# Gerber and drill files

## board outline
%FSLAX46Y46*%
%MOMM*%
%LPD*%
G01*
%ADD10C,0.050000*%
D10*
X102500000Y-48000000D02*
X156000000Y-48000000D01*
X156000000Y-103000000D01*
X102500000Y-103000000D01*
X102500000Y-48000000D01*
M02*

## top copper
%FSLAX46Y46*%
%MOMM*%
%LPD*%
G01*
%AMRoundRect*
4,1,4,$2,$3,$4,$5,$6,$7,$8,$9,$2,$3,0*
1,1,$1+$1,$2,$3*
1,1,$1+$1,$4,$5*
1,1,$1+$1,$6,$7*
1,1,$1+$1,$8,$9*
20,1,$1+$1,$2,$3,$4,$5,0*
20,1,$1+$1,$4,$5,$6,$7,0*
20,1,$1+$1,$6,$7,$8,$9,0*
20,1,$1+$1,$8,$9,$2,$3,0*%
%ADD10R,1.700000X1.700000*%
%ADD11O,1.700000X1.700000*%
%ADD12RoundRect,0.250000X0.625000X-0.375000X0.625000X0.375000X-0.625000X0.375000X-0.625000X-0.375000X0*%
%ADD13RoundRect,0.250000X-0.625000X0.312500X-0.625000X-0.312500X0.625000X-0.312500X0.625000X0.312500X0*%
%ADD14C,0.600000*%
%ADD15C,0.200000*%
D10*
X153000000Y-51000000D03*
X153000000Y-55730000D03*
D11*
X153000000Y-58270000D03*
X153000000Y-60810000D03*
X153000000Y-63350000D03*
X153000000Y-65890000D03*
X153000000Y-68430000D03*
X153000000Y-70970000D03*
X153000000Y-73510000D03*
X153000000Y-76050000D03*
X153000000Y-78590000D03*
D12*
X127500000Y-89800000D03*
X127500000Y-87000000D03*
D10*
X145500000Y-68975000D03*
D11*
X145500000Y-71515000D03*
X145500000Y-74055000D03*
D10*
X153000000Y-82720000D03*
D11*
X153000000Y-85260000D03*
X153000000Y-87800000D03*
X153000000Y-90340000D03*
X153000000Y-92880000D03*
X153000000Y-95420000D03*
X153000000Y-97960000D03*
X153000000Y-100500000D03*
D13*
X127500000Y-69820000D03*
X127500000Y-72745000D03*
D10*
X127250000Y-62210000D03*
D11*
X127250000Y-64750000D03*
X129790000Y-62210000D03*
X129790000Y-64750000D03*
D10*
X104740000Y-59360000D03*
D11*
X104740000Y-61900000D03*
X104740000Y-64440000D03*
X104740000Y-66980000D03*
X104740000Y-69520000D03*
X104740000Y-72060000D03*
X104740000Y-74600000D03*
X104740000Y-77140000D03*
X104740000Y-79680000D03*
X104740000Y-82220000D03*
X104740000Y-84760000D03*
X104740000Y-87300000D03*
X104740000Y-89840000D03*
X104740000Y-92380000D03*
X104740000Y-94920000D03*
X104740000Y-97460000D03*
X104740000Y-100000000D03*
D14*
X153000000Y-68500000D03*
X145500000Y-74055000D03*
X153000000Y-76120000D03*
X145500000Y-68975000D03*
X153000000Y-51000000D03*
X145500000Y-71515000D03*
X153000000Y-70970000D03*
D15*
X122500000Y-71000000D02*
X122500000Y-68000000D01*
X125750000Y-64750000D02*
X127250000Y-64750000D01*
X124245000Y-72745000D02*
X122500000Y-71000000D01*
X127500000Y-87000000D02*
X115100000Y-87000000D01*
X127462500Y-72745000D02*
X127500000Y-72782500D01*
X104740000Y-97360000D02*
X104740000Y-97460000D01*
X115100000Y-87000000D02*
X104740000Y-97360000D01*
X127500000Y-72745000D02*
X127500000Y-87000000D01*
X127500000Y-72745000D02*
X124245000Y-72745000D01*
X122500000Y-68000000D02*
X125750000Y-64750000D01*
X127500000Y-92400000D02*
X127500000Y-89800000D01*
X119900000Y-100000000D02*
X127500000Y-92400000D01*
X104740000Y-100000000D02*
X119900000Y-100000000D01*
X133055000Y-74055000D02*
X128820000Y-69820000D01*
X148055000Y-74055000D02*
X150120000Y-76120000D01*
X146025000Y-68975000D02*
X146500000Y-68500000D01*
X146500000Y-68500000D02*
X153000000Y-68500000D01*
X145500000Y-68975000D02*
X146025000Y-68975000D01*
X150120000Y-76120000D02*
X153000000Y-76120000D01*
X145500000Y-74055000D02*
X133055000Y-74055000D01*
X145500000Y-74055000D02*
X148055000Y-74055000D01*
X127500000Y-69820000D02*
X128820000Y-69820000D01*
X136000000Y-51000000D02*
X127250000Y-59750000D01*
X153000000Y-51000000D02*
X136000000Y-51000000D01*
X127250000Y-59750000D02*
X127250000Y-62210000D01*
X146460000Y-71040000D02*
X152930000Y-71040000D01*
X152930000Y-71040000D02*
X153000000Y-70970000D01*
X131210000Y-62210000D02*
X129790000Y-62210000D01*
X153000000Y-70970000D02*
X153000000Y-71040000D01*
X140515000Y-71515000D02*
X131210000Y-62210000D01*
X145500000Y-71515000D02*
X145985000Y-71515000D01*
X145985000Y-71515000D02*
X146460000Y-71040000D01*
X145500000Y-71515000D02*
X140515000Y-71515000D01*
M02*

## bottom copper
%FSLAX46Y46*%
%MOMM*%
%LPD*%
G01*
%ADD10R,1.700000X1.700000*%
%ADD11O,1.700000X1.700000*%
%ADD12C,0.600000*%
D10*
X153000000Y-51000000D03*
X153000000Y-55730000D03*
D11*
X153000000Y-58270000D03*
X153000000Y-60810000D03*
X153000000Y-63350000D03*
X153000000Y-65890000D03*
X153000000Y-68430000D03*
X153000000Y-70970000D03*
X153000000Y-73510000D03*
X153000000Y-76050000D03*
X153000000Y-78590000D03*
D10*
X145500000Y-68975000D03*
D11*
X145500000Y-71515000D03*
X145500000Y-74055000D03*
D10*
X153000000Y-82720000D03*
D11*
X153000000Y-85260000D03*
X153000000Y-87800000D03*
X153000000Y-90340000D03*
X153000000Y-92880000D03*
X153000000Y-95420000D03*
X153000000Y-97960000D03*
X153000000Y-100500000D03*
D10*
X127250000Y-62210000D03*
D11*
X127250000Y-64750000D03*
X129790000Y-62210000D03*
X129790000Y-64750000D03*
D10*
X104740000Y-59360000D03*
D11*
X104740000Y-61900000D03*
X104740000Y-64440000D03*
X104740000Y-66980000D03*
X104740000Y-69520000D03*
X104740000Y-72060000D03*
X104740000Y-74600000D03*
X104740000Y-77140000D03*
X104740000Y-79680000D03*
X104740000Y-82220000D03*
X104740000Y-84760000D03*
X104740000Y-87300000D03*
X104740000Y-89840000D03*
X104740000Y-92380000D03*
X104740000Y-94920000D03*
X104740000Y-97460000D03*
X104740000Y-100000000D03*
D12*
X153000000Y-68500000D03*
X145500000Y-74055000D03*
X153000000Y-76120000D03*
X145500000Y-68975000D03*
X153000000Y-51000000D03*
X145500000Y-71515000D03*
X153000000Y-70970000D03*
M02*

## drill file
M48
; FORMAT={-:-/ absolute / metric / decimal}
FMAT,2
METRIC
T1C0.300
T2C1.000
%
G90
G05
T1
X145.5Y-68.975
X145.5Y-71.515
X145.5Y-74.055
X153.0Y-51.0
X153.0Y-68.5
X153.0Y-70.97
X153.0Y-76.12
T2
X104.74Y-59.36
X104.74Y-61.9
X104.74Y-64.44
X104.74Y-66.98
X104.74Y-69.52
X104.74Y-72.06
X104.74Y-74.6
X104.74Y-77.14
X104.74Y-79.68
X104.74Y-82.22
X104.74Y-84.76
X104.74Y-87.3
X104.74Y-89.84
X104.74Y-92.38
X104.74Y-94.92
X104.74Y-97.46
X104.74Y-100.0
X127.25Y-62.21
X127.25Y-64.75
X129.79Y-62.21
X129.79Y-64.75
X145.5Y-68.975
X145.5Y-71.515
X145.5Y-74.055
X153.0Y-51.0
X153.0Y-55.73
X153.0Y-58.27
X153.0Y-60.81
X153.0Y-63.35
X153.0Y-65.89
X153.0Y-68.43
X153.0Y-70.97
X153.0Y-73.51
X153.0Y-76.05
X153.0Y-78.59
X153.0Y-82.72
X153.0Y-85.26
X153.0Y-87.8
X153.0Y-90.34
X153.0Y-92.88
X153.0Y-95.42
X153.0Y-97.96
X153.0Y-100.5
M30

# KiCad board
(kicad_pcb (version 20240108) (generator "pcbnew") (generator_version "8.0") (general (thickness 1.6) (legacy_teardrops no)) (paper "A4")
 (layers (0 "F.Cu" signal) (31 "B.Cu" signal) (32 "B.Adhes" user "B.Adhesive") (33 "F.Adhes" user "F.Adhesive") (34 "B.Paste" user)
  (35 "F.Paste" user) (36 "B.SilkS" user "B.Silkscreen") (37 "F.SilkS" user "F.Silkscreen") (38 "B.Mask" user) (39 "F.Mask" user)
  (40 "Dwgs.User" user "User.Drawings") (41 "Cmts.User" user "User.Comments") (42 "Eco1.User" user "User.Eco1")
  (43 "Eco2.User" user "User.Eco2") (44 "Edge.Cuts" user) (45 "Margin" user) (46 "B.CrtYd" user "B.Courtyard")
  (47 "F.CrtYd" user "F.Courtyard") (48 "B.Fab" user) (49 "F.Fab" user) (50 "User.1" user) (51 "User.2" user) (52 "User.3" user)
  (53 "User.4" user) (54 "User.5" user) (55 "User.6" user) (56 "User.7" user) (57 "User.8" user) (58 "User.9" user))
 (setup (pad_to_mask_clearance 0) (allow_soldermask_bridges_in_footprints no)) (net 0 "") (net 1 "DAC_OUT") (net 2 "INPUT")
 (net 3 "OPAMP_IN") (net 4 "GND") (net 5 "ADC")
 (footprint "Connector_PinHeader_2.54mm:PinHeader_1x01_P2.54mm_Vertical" (layer "F.Cu") (at 153 51)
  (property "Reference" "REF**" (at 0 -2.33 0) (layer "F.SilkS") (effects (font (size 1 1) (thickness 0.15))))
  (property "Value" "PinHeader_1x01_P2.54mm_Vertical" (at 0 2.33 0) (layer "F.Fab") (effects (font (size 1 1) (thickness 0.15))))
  (pad "1" thru_hole rect (at 0 0) (size 1.7 1.7) (drill 1) (layers "*.Cu" "*.Mask") (remove_unused_layers no) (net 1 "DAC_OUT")))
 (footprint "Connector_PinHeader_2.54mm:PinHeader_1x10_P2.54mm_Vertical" (layer "F.Cu") (at 153 55.73)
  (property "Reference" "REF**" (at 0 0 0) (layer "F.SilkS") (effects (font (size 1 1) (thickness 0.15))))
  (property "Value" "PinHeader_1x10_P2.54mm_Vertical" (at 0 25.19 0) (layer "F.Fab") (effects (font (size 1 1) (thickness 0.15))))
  (pad "1" thru_hole rect (at 0 0) (size 1.7 1.7) (drill 1) (layers "*.Cu" "*.Mask") (remove_unused_layers no))
  (pad "2" thru_hole oval (at 0 2.54) (size 1.7 1.7) (drill 1) (layers "*.Cu" "*.Mask") (remove_unused_layers no))
  (pad "3" thru_hole oval (at 0 5.08) (size 1.7 1.7) (drill 1) (layers "*.Cu" "*.Mask") (remove_unused_layers no))
  (pad "4" thru_hole oval (at 0 7.62) (size 1.7 1.7) (drill 1) (layers "*.Cu" "*.Mask") (remove_unused_layers no))
  (pad "5" thru_hole oval (at 0 10.16) (size 1.7 1.7) (drill 1) (layers "*.Cu" "*.Mask") (remove_unused_layers no))
  (pad "6" thru_hole oval (at 0 12.7) (size 1.7 1.7) (drill 1) (layers "*.Cu" "*.Mask") (remove_unused_layers no) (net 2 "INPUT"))
  (pad "7" thru_hole oval (at 0 15.24) (size 1.7 1.7) (drill 1) (layers "*.Cu" "*.Mask") (remove_unused_layers no) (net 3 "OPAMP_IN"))
  (pad "8" thru_hole oval (at 0 17.78) (size 1.7 1.7) (drill 1) (layers "*.Cu" "*.Mask") (remove_unused_layers no))
  (pad "9" thru_hole oval (at 0 20.32) (size 1.7 1.7) (drill 1) (layers "*.Cu" "*.Mask") (remove_unused_layers no) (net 2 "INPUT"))
  (pad "10" thru_hole oval (at 0 22.86) (size 1.7 1.7) (drill 1) (layers "*.Cu" "*.Mask") (remove_unused_layers no)))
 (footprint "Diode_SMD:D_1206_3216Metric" (layer "F.Cu") (at 127.5 88.4 90)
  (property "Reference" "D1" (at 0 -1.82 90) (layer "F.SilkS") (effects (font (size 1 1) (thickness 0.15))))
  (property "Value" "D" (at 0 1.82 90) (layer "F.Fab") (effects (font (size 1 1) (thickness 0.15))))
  (pad "1" smd roundrect (at -1.4 0 90) (size 1.25 1.75) (layers "F.Cu" "F.Paste" "F.Mask") (roundrect_rratio 0.2) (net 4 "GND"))
  (pad "2" smd roundrect (at 1.4 0 90) (size 1.25 1.75) (layers "F.Cu" "F.Paste" "F.Mask") (roundrect_rratio 0.2) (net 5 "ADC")))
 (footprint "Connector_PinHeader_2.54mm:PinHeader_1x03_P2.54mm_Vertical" (layer "F.Cu") (at 145.5 68.975)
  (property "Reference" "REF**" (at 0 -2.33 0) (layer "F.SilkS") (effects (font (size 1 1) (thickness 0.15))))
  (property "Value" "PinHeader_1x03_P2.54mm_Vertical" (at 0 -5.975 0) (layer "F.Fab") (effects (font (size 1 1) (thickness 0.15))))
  (pad "1" thru_hole rect (at 0 0) (size 1.7 1.7) (drill 1) (layers "*.Cu" "*.Mask") (remove_unused_layers no) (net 2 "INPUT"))
  (pad "2" thru_hole oval (at 0 2.54) (size 1.7 1.7) (drill 1) (layers "*.Cu" "*.Mask") (remove_unused_layers no) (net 3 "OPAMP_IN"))
  (pad "3" thru_hole oval (at 0 5.08) (size 1.7 1.7) (drill 1) (layers "*.Cu" "*.Mask") (remove_unused_layers no) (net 2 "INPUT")))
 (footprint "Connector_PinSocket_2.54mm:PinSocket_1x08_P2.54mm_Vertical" (layer "F.Cu") (at 153 82.72)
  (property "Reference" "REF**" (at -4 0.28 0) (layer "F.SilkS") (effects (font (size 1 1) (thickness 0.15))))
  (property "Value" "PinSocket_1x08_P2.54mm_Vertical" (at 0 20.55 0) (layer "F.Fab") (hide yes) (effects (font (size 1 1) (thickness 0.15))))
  (pad "1" thru_hole rect (at 0 0) (size 1.7 1.7) (drill 1) (layers "*.Cu" "*.Mask") (remove_unused_layers no))
  (pad "2" thru_hole oval (at 0 2.54) (size 1.7 1.7) (drill 1) (layers "*.Cu" "*.Mask") (remove_unused_layers no))
  (pad "3" thru_hole oval (at 0 5.08) (size 1.7 1.7) (drill 1) (layers "*.Cu" "*.Mask") (remove_unused_layers no))
  (pad "4" thru_hole oval (at 0 7.62) (size 1.7 1.7) (drill 1) (layers "*.Cu" "*.Mask") (remove_unused_layers no))
  (pad "5" thru_hole oval (at 0 10.16) (size 1.7 1.7) (drill 1) (layers "*.Cu" "*.Mask") (remove_unused_layers no))
  (pad "6" thru_hole oval (at 0 12.7) (size 1.7 1.7) (drill 1) (layers "*.Cu" "*.Mask") (remove_unused_layers no))
  (pad "7" thru_hole oval (at 0 15.24) (size 1.7 1.7) (drill 1) (layers "*.Cu" "*.Mask") (remove_unused_layers no))
  (pad "8" thru_hole oval (at 0 17.78) (size 1.7 1.7) (drill 1) (layers "*.Cu" "*.Mask") (remove_unused_layers no)))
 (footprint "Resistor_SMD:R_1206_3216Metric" (layer "F.Cu") (at 127.5 71.2825 -90)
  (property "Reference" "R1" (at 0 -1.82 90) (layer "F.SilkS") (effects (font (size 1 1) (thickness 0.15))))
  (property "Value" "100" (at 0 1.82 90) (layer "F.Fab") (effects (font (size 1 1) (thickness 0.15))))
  (pad "1" smd roundrect (at -1.4625 0 270) (size 1.125 1.75) (layers "F.Cu" "F.Paste" "F.Mask") (roundrect_rratio 0.222222) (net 2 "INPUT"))
  (pad "2" smd roundrect (at 1.4625 0 270) (size 1.125 1.75) (layers "F.Cu" "F.Paste" "F.Mask") (roundrect_rratio 0.222222) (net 5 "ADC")))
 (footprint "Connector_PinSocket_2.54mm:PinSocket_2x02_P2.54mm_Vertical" (layer "F.Cu") (at 127.25 62.21 90)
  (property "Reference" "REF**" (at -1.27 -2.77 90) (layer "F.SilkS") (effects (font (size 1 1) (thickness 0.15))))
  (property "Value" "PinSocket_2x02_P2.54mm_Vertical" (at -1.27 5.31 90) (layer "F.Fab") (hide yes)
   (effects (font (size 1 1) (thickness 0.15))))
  (pad "1" thru_hole rect (at 0 0 90) (size 1.7 1.7) (drill 1) (layers "*.Cu" "*.Mask") (remove_unused_layers no) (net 1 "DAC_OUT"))
  (pad "2" thru_hole oval (at -2.54 0 90) (size 1.7 1.7) (drill 1) (layers "*.Cu" "*.Mask") (remove_unused_layers no) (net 5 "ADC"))
  (pad "3" thru_hole oval (at 0 2.54 90) (size 1.7 1.7) (drill 1) (layers "*.Cu" "*.Mask") (remove_unused_layers no) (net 3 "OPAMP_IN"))
  (pad "4" thru_hole oval (at -2.54 2.54 90) (size 1.7 1.7) (drill 1) (layers "*.Cu" "*.Mask") (remove_unused_layers no)))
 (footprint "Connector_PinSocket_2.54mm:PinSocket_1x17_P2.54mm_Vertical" (layer "F.Cu") (at 104.74 59.36)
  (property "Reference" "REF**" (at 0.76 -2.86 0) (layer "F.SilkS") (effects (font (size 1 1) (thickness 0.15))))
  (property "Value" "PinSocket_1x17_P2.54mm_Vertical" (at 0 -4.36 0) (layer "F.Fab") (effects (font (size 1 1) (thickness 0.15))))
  (pad "1" thru_hole rect (at 0 0) (size 1.7 1.7) (drill 1) (layers "*.Cu" "*.Mask") (remove_unused_layers no))
  (pad "2" thru_hole oval (at 0 2.54) (size 1.7 1.7) (drill 1) (layers "*.Cu" "*.Mask") (remove_unused_layers no))
  (pad "3" thru_hole oval (at 0 5.08) (size 1.7 1.7) (drill 1) (layers "*.Cu" "*.Mask") (remove_unused_layers no))
  (pad "4" thru_hole oval (at 0 7.62) (size 1.7 1.7) (drill 1) (layers "*.Cu" "*.Mask") (remove_unused_layers no))
  (pad "5" thru_hole oval (at 0 10.16) (size 1.7 1.7) (drill 1) (layers "*.Cu" "*.Mask") (remove_unused_layers no))
  (pad "6" thru_hole oval (at 0 12.7) (size 1.7 1.7) (drill 1) (layers "*.Cu" "*.Mask") (remove_unused_layers no))
  (pad "7" thru_hole oval (at 0 15.24) (size 1.7 1.7) (drill 1) (layers "*.Cu" "*.Mask") (remove_unused_layers no))
  (pad "8" thru_hole oval (at 0 17.78) (size 1.7 1.7) (drill 1) (layers "*.Cu" "*.Mask") (remove_unused_layers no))
  (pad "9" thru_hole oval (at 0 20.32) (size 1.7 1.7) (drill 1) (layers "*.Cu" "*.Mask") (remove_unused_layers no))
  (pad "10" thru_hole oval (at 0 22.86) (size 1.7 1.7) (drill 1) (layers "*.Cu" "*.Mask") (remove_unused_layers no))
  (pad "11" thru_hole oval (at 0 25.4) (size 1.7 1.7) (drill 1) (layers "*.Cu" "*.Mask") (remove_unused_layers no))
  (pad "12" thru_hole oval (at 0 27.94) (size 1.7 1.7) (drill 1) (layers "*.Cu" "*.Mask") (remove_unused_layers no))
  (pad "13" thru_hole oval (at 0 30.48) (size 1.7 1.7) (drill 1) (layers "*.Cu" "*.Mask") (remove_unused_layers no))
  (pad "14" thru_hole oval (at 0 33.02) (size 1.7 1.7) (drill 1) (layers "*.Cu" "*.Mask") (remove_unused_layers no))
  (pad "15" thru_hole oval (at 0 35.56) (size 1.7 1.7) (drill 1) (layers "*.Cu" "*.Mask") (remove_unused_layers no))
  (pad "16" thru_hole oval (at 0 38.1) (size 1.7 1.7) (drill 1) (layers "*.Cu" "*.Mask") (remove_unused_layers no) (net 5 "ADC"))
  (pad "17" thru_hole oval (at 0 40.64) (size 1.7 1.7) (drill 1) (layers "*.Cu" "*.Mask") (remove_unused_layers no) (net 4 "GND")))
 (gr_rect (start 102.5 48) (end 156 103) (stroke (width 0.05) (type default)) (fill none) (layer "Edge.Cuts"))
 (segment (start 122.5 71) (end 122.5 68) (width 0.2) (layer "F.Cu") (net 5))
 (segment (start 125.75 64.75) (end 127.25 64.75) (width 0.2) (layer "F.Cu") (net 5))
 (segment (start 124.245 72.745) (end 122.5 71) (width 0.2) (layer "F.Cu") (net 5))
 (segment (start 127.5 87) (end 115.1 87) (width 0.2) (layer "F.Cu") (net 5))
 (segment (start 127.4625 72.745) (end 127.5 72.7825) (width 0.2) (layer "F.Cu") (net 5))
 (segment (start 104.74 97.36) (end 104.74 97.46) (width 0.2) (layer "F.Cu") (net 5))
 (segment (start 115.1 87) (end 104.74 97.36) (width 0.2) (layer "F.Cu") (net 5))
 (segment (start 127.5 72.745) (end 127.5 87) (width 0.2) (layer "F.Cu") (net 5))
 (segment (start 127.5 72.745) (end 124.245 72.745) (width 0.2) (layer "F.Cu") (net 5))
 (segment (start 122.5 68) (end 125.75 64.75) (width 0.2) (layer "F.Cu") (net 5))
 (segment (start 127.5 92.4) (end 127.5 89.8) (width 0.2) (layer "F.Cu") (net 4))
 (segment (start 119.9 100) (end 127.5 92.4) (width 0.2) (layer "F.Cu") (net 4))
 (segment (start 104.74 100) (end 119.9 100) (width 0.2) (layer "F.Cu") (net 4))
 (segment (start 133.055 74.055) (end 128.82 69.82) (width 0.2) (layer "F.Cu") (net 2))
 (segment (start 148.055 74.055) (end 150.12 76.12) (width 0.2) (layer "F.Cu") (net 2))
 (segment (start 146.025 68.975) (end 146.5 68.5) (width 0.2) (layer "F.Cu") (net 2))
 (segment (start 146.5 68.5) (end 153 68.5) (width 0.2) (layer "F.Cu") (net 2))
 (segment (start 145.5 68.975) (end 146.025 68.975) (width 0.2) (layer "F.Cu") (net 2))
 (segment (start 150.12 76.12) (end 153 76.12) (width 0.2) (layer "F.Cu") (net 2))
 (segment (start 145.5 74.055) (end 133.055 74.055) (width 0.2) (layer "F.Cu") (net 2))
 (segment (start 145.5 74.055) (end 148.055 74.055) (width 0.2) (layer "F.Cu") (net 2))
 (segment (start 127.5 69.82) (end 128.82 69.82) (width 0.2) (layer "F.Cu") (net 2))
 (via (at 153 68.5) (size 0.6) (drill 0.3) (layers "F.Cu" "B.Cu") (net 2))
 (via (at 145.5 74.055) (size 0.6) (drill 0.3) (layers "F.Cu" "B.Cu") (free yes) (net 2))
 (via (at 153 76.12) (size 0.6) (drill 0.3) (layers "F.Cu" "B.Cu") (free yes) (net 2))
 (via (at 145.5 68.975) (size 0.6) (drill 0.3) (layers "F.Cu" "B.Cu") (free yes) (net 2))
 (segment (start 136 51) (end 127.25 59.75) (width 0.2) (layer "F.Cu") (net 1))
 (segment (start 153 51) (end 136 51) (width 0.2) (layer "F.Cu") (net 1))
 (segment (start 127.25 59.75) (end 127.25 62.21) (width 0.2) (layer "F.Cu") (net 1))
 (via (at 153 51) (size 0.6) (drill 0.3) (layers "F.Cu" "B.Cu") (free yes) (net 1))
 (segment (start 146.46 71.04) (end 152.93 71.04) (width 0.2) (layer "F.Cu") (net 3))
 (segment (start 152.93 71.04) (end 153 70.97) (width 0.2) (layer "F.Cu") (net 3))
 (segment (start 131.21 62.21) (end 129.79 62.21) (width 0.2) (layer "F.Cu") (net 3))
 (segment (start 153 70.97) (end 153 71.04) (width 0.2) (layer "F.Cu") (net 3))
 (segment (start 140.515 71.515) (end 131.21 62.21) (width 0.2) (layer "F.Cu") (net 3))
 (segment (start 145.5 71.515) (end 145.985 71.515) (width 0.2) (layer "F.Cu") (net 3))
 (segment (start 145.985 71.515) (end 146.46 71.04) (width 0.2) (layer "F.Cu") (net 3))
 (segment (start 145.5 71.515) (end 140.515 71.515) (width 0.2) (layer "F.Cu") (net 3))
 (via (at 145.5 71.515) (size 0.6) (drill 0.3) (layers "F.Cu" "B.Cu") (free yes) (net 3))
 (via (at 153 70.97) (size 0.6) (drill 0.3) (layers "F.Cu" "B.Cu") (free yes) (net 3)))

